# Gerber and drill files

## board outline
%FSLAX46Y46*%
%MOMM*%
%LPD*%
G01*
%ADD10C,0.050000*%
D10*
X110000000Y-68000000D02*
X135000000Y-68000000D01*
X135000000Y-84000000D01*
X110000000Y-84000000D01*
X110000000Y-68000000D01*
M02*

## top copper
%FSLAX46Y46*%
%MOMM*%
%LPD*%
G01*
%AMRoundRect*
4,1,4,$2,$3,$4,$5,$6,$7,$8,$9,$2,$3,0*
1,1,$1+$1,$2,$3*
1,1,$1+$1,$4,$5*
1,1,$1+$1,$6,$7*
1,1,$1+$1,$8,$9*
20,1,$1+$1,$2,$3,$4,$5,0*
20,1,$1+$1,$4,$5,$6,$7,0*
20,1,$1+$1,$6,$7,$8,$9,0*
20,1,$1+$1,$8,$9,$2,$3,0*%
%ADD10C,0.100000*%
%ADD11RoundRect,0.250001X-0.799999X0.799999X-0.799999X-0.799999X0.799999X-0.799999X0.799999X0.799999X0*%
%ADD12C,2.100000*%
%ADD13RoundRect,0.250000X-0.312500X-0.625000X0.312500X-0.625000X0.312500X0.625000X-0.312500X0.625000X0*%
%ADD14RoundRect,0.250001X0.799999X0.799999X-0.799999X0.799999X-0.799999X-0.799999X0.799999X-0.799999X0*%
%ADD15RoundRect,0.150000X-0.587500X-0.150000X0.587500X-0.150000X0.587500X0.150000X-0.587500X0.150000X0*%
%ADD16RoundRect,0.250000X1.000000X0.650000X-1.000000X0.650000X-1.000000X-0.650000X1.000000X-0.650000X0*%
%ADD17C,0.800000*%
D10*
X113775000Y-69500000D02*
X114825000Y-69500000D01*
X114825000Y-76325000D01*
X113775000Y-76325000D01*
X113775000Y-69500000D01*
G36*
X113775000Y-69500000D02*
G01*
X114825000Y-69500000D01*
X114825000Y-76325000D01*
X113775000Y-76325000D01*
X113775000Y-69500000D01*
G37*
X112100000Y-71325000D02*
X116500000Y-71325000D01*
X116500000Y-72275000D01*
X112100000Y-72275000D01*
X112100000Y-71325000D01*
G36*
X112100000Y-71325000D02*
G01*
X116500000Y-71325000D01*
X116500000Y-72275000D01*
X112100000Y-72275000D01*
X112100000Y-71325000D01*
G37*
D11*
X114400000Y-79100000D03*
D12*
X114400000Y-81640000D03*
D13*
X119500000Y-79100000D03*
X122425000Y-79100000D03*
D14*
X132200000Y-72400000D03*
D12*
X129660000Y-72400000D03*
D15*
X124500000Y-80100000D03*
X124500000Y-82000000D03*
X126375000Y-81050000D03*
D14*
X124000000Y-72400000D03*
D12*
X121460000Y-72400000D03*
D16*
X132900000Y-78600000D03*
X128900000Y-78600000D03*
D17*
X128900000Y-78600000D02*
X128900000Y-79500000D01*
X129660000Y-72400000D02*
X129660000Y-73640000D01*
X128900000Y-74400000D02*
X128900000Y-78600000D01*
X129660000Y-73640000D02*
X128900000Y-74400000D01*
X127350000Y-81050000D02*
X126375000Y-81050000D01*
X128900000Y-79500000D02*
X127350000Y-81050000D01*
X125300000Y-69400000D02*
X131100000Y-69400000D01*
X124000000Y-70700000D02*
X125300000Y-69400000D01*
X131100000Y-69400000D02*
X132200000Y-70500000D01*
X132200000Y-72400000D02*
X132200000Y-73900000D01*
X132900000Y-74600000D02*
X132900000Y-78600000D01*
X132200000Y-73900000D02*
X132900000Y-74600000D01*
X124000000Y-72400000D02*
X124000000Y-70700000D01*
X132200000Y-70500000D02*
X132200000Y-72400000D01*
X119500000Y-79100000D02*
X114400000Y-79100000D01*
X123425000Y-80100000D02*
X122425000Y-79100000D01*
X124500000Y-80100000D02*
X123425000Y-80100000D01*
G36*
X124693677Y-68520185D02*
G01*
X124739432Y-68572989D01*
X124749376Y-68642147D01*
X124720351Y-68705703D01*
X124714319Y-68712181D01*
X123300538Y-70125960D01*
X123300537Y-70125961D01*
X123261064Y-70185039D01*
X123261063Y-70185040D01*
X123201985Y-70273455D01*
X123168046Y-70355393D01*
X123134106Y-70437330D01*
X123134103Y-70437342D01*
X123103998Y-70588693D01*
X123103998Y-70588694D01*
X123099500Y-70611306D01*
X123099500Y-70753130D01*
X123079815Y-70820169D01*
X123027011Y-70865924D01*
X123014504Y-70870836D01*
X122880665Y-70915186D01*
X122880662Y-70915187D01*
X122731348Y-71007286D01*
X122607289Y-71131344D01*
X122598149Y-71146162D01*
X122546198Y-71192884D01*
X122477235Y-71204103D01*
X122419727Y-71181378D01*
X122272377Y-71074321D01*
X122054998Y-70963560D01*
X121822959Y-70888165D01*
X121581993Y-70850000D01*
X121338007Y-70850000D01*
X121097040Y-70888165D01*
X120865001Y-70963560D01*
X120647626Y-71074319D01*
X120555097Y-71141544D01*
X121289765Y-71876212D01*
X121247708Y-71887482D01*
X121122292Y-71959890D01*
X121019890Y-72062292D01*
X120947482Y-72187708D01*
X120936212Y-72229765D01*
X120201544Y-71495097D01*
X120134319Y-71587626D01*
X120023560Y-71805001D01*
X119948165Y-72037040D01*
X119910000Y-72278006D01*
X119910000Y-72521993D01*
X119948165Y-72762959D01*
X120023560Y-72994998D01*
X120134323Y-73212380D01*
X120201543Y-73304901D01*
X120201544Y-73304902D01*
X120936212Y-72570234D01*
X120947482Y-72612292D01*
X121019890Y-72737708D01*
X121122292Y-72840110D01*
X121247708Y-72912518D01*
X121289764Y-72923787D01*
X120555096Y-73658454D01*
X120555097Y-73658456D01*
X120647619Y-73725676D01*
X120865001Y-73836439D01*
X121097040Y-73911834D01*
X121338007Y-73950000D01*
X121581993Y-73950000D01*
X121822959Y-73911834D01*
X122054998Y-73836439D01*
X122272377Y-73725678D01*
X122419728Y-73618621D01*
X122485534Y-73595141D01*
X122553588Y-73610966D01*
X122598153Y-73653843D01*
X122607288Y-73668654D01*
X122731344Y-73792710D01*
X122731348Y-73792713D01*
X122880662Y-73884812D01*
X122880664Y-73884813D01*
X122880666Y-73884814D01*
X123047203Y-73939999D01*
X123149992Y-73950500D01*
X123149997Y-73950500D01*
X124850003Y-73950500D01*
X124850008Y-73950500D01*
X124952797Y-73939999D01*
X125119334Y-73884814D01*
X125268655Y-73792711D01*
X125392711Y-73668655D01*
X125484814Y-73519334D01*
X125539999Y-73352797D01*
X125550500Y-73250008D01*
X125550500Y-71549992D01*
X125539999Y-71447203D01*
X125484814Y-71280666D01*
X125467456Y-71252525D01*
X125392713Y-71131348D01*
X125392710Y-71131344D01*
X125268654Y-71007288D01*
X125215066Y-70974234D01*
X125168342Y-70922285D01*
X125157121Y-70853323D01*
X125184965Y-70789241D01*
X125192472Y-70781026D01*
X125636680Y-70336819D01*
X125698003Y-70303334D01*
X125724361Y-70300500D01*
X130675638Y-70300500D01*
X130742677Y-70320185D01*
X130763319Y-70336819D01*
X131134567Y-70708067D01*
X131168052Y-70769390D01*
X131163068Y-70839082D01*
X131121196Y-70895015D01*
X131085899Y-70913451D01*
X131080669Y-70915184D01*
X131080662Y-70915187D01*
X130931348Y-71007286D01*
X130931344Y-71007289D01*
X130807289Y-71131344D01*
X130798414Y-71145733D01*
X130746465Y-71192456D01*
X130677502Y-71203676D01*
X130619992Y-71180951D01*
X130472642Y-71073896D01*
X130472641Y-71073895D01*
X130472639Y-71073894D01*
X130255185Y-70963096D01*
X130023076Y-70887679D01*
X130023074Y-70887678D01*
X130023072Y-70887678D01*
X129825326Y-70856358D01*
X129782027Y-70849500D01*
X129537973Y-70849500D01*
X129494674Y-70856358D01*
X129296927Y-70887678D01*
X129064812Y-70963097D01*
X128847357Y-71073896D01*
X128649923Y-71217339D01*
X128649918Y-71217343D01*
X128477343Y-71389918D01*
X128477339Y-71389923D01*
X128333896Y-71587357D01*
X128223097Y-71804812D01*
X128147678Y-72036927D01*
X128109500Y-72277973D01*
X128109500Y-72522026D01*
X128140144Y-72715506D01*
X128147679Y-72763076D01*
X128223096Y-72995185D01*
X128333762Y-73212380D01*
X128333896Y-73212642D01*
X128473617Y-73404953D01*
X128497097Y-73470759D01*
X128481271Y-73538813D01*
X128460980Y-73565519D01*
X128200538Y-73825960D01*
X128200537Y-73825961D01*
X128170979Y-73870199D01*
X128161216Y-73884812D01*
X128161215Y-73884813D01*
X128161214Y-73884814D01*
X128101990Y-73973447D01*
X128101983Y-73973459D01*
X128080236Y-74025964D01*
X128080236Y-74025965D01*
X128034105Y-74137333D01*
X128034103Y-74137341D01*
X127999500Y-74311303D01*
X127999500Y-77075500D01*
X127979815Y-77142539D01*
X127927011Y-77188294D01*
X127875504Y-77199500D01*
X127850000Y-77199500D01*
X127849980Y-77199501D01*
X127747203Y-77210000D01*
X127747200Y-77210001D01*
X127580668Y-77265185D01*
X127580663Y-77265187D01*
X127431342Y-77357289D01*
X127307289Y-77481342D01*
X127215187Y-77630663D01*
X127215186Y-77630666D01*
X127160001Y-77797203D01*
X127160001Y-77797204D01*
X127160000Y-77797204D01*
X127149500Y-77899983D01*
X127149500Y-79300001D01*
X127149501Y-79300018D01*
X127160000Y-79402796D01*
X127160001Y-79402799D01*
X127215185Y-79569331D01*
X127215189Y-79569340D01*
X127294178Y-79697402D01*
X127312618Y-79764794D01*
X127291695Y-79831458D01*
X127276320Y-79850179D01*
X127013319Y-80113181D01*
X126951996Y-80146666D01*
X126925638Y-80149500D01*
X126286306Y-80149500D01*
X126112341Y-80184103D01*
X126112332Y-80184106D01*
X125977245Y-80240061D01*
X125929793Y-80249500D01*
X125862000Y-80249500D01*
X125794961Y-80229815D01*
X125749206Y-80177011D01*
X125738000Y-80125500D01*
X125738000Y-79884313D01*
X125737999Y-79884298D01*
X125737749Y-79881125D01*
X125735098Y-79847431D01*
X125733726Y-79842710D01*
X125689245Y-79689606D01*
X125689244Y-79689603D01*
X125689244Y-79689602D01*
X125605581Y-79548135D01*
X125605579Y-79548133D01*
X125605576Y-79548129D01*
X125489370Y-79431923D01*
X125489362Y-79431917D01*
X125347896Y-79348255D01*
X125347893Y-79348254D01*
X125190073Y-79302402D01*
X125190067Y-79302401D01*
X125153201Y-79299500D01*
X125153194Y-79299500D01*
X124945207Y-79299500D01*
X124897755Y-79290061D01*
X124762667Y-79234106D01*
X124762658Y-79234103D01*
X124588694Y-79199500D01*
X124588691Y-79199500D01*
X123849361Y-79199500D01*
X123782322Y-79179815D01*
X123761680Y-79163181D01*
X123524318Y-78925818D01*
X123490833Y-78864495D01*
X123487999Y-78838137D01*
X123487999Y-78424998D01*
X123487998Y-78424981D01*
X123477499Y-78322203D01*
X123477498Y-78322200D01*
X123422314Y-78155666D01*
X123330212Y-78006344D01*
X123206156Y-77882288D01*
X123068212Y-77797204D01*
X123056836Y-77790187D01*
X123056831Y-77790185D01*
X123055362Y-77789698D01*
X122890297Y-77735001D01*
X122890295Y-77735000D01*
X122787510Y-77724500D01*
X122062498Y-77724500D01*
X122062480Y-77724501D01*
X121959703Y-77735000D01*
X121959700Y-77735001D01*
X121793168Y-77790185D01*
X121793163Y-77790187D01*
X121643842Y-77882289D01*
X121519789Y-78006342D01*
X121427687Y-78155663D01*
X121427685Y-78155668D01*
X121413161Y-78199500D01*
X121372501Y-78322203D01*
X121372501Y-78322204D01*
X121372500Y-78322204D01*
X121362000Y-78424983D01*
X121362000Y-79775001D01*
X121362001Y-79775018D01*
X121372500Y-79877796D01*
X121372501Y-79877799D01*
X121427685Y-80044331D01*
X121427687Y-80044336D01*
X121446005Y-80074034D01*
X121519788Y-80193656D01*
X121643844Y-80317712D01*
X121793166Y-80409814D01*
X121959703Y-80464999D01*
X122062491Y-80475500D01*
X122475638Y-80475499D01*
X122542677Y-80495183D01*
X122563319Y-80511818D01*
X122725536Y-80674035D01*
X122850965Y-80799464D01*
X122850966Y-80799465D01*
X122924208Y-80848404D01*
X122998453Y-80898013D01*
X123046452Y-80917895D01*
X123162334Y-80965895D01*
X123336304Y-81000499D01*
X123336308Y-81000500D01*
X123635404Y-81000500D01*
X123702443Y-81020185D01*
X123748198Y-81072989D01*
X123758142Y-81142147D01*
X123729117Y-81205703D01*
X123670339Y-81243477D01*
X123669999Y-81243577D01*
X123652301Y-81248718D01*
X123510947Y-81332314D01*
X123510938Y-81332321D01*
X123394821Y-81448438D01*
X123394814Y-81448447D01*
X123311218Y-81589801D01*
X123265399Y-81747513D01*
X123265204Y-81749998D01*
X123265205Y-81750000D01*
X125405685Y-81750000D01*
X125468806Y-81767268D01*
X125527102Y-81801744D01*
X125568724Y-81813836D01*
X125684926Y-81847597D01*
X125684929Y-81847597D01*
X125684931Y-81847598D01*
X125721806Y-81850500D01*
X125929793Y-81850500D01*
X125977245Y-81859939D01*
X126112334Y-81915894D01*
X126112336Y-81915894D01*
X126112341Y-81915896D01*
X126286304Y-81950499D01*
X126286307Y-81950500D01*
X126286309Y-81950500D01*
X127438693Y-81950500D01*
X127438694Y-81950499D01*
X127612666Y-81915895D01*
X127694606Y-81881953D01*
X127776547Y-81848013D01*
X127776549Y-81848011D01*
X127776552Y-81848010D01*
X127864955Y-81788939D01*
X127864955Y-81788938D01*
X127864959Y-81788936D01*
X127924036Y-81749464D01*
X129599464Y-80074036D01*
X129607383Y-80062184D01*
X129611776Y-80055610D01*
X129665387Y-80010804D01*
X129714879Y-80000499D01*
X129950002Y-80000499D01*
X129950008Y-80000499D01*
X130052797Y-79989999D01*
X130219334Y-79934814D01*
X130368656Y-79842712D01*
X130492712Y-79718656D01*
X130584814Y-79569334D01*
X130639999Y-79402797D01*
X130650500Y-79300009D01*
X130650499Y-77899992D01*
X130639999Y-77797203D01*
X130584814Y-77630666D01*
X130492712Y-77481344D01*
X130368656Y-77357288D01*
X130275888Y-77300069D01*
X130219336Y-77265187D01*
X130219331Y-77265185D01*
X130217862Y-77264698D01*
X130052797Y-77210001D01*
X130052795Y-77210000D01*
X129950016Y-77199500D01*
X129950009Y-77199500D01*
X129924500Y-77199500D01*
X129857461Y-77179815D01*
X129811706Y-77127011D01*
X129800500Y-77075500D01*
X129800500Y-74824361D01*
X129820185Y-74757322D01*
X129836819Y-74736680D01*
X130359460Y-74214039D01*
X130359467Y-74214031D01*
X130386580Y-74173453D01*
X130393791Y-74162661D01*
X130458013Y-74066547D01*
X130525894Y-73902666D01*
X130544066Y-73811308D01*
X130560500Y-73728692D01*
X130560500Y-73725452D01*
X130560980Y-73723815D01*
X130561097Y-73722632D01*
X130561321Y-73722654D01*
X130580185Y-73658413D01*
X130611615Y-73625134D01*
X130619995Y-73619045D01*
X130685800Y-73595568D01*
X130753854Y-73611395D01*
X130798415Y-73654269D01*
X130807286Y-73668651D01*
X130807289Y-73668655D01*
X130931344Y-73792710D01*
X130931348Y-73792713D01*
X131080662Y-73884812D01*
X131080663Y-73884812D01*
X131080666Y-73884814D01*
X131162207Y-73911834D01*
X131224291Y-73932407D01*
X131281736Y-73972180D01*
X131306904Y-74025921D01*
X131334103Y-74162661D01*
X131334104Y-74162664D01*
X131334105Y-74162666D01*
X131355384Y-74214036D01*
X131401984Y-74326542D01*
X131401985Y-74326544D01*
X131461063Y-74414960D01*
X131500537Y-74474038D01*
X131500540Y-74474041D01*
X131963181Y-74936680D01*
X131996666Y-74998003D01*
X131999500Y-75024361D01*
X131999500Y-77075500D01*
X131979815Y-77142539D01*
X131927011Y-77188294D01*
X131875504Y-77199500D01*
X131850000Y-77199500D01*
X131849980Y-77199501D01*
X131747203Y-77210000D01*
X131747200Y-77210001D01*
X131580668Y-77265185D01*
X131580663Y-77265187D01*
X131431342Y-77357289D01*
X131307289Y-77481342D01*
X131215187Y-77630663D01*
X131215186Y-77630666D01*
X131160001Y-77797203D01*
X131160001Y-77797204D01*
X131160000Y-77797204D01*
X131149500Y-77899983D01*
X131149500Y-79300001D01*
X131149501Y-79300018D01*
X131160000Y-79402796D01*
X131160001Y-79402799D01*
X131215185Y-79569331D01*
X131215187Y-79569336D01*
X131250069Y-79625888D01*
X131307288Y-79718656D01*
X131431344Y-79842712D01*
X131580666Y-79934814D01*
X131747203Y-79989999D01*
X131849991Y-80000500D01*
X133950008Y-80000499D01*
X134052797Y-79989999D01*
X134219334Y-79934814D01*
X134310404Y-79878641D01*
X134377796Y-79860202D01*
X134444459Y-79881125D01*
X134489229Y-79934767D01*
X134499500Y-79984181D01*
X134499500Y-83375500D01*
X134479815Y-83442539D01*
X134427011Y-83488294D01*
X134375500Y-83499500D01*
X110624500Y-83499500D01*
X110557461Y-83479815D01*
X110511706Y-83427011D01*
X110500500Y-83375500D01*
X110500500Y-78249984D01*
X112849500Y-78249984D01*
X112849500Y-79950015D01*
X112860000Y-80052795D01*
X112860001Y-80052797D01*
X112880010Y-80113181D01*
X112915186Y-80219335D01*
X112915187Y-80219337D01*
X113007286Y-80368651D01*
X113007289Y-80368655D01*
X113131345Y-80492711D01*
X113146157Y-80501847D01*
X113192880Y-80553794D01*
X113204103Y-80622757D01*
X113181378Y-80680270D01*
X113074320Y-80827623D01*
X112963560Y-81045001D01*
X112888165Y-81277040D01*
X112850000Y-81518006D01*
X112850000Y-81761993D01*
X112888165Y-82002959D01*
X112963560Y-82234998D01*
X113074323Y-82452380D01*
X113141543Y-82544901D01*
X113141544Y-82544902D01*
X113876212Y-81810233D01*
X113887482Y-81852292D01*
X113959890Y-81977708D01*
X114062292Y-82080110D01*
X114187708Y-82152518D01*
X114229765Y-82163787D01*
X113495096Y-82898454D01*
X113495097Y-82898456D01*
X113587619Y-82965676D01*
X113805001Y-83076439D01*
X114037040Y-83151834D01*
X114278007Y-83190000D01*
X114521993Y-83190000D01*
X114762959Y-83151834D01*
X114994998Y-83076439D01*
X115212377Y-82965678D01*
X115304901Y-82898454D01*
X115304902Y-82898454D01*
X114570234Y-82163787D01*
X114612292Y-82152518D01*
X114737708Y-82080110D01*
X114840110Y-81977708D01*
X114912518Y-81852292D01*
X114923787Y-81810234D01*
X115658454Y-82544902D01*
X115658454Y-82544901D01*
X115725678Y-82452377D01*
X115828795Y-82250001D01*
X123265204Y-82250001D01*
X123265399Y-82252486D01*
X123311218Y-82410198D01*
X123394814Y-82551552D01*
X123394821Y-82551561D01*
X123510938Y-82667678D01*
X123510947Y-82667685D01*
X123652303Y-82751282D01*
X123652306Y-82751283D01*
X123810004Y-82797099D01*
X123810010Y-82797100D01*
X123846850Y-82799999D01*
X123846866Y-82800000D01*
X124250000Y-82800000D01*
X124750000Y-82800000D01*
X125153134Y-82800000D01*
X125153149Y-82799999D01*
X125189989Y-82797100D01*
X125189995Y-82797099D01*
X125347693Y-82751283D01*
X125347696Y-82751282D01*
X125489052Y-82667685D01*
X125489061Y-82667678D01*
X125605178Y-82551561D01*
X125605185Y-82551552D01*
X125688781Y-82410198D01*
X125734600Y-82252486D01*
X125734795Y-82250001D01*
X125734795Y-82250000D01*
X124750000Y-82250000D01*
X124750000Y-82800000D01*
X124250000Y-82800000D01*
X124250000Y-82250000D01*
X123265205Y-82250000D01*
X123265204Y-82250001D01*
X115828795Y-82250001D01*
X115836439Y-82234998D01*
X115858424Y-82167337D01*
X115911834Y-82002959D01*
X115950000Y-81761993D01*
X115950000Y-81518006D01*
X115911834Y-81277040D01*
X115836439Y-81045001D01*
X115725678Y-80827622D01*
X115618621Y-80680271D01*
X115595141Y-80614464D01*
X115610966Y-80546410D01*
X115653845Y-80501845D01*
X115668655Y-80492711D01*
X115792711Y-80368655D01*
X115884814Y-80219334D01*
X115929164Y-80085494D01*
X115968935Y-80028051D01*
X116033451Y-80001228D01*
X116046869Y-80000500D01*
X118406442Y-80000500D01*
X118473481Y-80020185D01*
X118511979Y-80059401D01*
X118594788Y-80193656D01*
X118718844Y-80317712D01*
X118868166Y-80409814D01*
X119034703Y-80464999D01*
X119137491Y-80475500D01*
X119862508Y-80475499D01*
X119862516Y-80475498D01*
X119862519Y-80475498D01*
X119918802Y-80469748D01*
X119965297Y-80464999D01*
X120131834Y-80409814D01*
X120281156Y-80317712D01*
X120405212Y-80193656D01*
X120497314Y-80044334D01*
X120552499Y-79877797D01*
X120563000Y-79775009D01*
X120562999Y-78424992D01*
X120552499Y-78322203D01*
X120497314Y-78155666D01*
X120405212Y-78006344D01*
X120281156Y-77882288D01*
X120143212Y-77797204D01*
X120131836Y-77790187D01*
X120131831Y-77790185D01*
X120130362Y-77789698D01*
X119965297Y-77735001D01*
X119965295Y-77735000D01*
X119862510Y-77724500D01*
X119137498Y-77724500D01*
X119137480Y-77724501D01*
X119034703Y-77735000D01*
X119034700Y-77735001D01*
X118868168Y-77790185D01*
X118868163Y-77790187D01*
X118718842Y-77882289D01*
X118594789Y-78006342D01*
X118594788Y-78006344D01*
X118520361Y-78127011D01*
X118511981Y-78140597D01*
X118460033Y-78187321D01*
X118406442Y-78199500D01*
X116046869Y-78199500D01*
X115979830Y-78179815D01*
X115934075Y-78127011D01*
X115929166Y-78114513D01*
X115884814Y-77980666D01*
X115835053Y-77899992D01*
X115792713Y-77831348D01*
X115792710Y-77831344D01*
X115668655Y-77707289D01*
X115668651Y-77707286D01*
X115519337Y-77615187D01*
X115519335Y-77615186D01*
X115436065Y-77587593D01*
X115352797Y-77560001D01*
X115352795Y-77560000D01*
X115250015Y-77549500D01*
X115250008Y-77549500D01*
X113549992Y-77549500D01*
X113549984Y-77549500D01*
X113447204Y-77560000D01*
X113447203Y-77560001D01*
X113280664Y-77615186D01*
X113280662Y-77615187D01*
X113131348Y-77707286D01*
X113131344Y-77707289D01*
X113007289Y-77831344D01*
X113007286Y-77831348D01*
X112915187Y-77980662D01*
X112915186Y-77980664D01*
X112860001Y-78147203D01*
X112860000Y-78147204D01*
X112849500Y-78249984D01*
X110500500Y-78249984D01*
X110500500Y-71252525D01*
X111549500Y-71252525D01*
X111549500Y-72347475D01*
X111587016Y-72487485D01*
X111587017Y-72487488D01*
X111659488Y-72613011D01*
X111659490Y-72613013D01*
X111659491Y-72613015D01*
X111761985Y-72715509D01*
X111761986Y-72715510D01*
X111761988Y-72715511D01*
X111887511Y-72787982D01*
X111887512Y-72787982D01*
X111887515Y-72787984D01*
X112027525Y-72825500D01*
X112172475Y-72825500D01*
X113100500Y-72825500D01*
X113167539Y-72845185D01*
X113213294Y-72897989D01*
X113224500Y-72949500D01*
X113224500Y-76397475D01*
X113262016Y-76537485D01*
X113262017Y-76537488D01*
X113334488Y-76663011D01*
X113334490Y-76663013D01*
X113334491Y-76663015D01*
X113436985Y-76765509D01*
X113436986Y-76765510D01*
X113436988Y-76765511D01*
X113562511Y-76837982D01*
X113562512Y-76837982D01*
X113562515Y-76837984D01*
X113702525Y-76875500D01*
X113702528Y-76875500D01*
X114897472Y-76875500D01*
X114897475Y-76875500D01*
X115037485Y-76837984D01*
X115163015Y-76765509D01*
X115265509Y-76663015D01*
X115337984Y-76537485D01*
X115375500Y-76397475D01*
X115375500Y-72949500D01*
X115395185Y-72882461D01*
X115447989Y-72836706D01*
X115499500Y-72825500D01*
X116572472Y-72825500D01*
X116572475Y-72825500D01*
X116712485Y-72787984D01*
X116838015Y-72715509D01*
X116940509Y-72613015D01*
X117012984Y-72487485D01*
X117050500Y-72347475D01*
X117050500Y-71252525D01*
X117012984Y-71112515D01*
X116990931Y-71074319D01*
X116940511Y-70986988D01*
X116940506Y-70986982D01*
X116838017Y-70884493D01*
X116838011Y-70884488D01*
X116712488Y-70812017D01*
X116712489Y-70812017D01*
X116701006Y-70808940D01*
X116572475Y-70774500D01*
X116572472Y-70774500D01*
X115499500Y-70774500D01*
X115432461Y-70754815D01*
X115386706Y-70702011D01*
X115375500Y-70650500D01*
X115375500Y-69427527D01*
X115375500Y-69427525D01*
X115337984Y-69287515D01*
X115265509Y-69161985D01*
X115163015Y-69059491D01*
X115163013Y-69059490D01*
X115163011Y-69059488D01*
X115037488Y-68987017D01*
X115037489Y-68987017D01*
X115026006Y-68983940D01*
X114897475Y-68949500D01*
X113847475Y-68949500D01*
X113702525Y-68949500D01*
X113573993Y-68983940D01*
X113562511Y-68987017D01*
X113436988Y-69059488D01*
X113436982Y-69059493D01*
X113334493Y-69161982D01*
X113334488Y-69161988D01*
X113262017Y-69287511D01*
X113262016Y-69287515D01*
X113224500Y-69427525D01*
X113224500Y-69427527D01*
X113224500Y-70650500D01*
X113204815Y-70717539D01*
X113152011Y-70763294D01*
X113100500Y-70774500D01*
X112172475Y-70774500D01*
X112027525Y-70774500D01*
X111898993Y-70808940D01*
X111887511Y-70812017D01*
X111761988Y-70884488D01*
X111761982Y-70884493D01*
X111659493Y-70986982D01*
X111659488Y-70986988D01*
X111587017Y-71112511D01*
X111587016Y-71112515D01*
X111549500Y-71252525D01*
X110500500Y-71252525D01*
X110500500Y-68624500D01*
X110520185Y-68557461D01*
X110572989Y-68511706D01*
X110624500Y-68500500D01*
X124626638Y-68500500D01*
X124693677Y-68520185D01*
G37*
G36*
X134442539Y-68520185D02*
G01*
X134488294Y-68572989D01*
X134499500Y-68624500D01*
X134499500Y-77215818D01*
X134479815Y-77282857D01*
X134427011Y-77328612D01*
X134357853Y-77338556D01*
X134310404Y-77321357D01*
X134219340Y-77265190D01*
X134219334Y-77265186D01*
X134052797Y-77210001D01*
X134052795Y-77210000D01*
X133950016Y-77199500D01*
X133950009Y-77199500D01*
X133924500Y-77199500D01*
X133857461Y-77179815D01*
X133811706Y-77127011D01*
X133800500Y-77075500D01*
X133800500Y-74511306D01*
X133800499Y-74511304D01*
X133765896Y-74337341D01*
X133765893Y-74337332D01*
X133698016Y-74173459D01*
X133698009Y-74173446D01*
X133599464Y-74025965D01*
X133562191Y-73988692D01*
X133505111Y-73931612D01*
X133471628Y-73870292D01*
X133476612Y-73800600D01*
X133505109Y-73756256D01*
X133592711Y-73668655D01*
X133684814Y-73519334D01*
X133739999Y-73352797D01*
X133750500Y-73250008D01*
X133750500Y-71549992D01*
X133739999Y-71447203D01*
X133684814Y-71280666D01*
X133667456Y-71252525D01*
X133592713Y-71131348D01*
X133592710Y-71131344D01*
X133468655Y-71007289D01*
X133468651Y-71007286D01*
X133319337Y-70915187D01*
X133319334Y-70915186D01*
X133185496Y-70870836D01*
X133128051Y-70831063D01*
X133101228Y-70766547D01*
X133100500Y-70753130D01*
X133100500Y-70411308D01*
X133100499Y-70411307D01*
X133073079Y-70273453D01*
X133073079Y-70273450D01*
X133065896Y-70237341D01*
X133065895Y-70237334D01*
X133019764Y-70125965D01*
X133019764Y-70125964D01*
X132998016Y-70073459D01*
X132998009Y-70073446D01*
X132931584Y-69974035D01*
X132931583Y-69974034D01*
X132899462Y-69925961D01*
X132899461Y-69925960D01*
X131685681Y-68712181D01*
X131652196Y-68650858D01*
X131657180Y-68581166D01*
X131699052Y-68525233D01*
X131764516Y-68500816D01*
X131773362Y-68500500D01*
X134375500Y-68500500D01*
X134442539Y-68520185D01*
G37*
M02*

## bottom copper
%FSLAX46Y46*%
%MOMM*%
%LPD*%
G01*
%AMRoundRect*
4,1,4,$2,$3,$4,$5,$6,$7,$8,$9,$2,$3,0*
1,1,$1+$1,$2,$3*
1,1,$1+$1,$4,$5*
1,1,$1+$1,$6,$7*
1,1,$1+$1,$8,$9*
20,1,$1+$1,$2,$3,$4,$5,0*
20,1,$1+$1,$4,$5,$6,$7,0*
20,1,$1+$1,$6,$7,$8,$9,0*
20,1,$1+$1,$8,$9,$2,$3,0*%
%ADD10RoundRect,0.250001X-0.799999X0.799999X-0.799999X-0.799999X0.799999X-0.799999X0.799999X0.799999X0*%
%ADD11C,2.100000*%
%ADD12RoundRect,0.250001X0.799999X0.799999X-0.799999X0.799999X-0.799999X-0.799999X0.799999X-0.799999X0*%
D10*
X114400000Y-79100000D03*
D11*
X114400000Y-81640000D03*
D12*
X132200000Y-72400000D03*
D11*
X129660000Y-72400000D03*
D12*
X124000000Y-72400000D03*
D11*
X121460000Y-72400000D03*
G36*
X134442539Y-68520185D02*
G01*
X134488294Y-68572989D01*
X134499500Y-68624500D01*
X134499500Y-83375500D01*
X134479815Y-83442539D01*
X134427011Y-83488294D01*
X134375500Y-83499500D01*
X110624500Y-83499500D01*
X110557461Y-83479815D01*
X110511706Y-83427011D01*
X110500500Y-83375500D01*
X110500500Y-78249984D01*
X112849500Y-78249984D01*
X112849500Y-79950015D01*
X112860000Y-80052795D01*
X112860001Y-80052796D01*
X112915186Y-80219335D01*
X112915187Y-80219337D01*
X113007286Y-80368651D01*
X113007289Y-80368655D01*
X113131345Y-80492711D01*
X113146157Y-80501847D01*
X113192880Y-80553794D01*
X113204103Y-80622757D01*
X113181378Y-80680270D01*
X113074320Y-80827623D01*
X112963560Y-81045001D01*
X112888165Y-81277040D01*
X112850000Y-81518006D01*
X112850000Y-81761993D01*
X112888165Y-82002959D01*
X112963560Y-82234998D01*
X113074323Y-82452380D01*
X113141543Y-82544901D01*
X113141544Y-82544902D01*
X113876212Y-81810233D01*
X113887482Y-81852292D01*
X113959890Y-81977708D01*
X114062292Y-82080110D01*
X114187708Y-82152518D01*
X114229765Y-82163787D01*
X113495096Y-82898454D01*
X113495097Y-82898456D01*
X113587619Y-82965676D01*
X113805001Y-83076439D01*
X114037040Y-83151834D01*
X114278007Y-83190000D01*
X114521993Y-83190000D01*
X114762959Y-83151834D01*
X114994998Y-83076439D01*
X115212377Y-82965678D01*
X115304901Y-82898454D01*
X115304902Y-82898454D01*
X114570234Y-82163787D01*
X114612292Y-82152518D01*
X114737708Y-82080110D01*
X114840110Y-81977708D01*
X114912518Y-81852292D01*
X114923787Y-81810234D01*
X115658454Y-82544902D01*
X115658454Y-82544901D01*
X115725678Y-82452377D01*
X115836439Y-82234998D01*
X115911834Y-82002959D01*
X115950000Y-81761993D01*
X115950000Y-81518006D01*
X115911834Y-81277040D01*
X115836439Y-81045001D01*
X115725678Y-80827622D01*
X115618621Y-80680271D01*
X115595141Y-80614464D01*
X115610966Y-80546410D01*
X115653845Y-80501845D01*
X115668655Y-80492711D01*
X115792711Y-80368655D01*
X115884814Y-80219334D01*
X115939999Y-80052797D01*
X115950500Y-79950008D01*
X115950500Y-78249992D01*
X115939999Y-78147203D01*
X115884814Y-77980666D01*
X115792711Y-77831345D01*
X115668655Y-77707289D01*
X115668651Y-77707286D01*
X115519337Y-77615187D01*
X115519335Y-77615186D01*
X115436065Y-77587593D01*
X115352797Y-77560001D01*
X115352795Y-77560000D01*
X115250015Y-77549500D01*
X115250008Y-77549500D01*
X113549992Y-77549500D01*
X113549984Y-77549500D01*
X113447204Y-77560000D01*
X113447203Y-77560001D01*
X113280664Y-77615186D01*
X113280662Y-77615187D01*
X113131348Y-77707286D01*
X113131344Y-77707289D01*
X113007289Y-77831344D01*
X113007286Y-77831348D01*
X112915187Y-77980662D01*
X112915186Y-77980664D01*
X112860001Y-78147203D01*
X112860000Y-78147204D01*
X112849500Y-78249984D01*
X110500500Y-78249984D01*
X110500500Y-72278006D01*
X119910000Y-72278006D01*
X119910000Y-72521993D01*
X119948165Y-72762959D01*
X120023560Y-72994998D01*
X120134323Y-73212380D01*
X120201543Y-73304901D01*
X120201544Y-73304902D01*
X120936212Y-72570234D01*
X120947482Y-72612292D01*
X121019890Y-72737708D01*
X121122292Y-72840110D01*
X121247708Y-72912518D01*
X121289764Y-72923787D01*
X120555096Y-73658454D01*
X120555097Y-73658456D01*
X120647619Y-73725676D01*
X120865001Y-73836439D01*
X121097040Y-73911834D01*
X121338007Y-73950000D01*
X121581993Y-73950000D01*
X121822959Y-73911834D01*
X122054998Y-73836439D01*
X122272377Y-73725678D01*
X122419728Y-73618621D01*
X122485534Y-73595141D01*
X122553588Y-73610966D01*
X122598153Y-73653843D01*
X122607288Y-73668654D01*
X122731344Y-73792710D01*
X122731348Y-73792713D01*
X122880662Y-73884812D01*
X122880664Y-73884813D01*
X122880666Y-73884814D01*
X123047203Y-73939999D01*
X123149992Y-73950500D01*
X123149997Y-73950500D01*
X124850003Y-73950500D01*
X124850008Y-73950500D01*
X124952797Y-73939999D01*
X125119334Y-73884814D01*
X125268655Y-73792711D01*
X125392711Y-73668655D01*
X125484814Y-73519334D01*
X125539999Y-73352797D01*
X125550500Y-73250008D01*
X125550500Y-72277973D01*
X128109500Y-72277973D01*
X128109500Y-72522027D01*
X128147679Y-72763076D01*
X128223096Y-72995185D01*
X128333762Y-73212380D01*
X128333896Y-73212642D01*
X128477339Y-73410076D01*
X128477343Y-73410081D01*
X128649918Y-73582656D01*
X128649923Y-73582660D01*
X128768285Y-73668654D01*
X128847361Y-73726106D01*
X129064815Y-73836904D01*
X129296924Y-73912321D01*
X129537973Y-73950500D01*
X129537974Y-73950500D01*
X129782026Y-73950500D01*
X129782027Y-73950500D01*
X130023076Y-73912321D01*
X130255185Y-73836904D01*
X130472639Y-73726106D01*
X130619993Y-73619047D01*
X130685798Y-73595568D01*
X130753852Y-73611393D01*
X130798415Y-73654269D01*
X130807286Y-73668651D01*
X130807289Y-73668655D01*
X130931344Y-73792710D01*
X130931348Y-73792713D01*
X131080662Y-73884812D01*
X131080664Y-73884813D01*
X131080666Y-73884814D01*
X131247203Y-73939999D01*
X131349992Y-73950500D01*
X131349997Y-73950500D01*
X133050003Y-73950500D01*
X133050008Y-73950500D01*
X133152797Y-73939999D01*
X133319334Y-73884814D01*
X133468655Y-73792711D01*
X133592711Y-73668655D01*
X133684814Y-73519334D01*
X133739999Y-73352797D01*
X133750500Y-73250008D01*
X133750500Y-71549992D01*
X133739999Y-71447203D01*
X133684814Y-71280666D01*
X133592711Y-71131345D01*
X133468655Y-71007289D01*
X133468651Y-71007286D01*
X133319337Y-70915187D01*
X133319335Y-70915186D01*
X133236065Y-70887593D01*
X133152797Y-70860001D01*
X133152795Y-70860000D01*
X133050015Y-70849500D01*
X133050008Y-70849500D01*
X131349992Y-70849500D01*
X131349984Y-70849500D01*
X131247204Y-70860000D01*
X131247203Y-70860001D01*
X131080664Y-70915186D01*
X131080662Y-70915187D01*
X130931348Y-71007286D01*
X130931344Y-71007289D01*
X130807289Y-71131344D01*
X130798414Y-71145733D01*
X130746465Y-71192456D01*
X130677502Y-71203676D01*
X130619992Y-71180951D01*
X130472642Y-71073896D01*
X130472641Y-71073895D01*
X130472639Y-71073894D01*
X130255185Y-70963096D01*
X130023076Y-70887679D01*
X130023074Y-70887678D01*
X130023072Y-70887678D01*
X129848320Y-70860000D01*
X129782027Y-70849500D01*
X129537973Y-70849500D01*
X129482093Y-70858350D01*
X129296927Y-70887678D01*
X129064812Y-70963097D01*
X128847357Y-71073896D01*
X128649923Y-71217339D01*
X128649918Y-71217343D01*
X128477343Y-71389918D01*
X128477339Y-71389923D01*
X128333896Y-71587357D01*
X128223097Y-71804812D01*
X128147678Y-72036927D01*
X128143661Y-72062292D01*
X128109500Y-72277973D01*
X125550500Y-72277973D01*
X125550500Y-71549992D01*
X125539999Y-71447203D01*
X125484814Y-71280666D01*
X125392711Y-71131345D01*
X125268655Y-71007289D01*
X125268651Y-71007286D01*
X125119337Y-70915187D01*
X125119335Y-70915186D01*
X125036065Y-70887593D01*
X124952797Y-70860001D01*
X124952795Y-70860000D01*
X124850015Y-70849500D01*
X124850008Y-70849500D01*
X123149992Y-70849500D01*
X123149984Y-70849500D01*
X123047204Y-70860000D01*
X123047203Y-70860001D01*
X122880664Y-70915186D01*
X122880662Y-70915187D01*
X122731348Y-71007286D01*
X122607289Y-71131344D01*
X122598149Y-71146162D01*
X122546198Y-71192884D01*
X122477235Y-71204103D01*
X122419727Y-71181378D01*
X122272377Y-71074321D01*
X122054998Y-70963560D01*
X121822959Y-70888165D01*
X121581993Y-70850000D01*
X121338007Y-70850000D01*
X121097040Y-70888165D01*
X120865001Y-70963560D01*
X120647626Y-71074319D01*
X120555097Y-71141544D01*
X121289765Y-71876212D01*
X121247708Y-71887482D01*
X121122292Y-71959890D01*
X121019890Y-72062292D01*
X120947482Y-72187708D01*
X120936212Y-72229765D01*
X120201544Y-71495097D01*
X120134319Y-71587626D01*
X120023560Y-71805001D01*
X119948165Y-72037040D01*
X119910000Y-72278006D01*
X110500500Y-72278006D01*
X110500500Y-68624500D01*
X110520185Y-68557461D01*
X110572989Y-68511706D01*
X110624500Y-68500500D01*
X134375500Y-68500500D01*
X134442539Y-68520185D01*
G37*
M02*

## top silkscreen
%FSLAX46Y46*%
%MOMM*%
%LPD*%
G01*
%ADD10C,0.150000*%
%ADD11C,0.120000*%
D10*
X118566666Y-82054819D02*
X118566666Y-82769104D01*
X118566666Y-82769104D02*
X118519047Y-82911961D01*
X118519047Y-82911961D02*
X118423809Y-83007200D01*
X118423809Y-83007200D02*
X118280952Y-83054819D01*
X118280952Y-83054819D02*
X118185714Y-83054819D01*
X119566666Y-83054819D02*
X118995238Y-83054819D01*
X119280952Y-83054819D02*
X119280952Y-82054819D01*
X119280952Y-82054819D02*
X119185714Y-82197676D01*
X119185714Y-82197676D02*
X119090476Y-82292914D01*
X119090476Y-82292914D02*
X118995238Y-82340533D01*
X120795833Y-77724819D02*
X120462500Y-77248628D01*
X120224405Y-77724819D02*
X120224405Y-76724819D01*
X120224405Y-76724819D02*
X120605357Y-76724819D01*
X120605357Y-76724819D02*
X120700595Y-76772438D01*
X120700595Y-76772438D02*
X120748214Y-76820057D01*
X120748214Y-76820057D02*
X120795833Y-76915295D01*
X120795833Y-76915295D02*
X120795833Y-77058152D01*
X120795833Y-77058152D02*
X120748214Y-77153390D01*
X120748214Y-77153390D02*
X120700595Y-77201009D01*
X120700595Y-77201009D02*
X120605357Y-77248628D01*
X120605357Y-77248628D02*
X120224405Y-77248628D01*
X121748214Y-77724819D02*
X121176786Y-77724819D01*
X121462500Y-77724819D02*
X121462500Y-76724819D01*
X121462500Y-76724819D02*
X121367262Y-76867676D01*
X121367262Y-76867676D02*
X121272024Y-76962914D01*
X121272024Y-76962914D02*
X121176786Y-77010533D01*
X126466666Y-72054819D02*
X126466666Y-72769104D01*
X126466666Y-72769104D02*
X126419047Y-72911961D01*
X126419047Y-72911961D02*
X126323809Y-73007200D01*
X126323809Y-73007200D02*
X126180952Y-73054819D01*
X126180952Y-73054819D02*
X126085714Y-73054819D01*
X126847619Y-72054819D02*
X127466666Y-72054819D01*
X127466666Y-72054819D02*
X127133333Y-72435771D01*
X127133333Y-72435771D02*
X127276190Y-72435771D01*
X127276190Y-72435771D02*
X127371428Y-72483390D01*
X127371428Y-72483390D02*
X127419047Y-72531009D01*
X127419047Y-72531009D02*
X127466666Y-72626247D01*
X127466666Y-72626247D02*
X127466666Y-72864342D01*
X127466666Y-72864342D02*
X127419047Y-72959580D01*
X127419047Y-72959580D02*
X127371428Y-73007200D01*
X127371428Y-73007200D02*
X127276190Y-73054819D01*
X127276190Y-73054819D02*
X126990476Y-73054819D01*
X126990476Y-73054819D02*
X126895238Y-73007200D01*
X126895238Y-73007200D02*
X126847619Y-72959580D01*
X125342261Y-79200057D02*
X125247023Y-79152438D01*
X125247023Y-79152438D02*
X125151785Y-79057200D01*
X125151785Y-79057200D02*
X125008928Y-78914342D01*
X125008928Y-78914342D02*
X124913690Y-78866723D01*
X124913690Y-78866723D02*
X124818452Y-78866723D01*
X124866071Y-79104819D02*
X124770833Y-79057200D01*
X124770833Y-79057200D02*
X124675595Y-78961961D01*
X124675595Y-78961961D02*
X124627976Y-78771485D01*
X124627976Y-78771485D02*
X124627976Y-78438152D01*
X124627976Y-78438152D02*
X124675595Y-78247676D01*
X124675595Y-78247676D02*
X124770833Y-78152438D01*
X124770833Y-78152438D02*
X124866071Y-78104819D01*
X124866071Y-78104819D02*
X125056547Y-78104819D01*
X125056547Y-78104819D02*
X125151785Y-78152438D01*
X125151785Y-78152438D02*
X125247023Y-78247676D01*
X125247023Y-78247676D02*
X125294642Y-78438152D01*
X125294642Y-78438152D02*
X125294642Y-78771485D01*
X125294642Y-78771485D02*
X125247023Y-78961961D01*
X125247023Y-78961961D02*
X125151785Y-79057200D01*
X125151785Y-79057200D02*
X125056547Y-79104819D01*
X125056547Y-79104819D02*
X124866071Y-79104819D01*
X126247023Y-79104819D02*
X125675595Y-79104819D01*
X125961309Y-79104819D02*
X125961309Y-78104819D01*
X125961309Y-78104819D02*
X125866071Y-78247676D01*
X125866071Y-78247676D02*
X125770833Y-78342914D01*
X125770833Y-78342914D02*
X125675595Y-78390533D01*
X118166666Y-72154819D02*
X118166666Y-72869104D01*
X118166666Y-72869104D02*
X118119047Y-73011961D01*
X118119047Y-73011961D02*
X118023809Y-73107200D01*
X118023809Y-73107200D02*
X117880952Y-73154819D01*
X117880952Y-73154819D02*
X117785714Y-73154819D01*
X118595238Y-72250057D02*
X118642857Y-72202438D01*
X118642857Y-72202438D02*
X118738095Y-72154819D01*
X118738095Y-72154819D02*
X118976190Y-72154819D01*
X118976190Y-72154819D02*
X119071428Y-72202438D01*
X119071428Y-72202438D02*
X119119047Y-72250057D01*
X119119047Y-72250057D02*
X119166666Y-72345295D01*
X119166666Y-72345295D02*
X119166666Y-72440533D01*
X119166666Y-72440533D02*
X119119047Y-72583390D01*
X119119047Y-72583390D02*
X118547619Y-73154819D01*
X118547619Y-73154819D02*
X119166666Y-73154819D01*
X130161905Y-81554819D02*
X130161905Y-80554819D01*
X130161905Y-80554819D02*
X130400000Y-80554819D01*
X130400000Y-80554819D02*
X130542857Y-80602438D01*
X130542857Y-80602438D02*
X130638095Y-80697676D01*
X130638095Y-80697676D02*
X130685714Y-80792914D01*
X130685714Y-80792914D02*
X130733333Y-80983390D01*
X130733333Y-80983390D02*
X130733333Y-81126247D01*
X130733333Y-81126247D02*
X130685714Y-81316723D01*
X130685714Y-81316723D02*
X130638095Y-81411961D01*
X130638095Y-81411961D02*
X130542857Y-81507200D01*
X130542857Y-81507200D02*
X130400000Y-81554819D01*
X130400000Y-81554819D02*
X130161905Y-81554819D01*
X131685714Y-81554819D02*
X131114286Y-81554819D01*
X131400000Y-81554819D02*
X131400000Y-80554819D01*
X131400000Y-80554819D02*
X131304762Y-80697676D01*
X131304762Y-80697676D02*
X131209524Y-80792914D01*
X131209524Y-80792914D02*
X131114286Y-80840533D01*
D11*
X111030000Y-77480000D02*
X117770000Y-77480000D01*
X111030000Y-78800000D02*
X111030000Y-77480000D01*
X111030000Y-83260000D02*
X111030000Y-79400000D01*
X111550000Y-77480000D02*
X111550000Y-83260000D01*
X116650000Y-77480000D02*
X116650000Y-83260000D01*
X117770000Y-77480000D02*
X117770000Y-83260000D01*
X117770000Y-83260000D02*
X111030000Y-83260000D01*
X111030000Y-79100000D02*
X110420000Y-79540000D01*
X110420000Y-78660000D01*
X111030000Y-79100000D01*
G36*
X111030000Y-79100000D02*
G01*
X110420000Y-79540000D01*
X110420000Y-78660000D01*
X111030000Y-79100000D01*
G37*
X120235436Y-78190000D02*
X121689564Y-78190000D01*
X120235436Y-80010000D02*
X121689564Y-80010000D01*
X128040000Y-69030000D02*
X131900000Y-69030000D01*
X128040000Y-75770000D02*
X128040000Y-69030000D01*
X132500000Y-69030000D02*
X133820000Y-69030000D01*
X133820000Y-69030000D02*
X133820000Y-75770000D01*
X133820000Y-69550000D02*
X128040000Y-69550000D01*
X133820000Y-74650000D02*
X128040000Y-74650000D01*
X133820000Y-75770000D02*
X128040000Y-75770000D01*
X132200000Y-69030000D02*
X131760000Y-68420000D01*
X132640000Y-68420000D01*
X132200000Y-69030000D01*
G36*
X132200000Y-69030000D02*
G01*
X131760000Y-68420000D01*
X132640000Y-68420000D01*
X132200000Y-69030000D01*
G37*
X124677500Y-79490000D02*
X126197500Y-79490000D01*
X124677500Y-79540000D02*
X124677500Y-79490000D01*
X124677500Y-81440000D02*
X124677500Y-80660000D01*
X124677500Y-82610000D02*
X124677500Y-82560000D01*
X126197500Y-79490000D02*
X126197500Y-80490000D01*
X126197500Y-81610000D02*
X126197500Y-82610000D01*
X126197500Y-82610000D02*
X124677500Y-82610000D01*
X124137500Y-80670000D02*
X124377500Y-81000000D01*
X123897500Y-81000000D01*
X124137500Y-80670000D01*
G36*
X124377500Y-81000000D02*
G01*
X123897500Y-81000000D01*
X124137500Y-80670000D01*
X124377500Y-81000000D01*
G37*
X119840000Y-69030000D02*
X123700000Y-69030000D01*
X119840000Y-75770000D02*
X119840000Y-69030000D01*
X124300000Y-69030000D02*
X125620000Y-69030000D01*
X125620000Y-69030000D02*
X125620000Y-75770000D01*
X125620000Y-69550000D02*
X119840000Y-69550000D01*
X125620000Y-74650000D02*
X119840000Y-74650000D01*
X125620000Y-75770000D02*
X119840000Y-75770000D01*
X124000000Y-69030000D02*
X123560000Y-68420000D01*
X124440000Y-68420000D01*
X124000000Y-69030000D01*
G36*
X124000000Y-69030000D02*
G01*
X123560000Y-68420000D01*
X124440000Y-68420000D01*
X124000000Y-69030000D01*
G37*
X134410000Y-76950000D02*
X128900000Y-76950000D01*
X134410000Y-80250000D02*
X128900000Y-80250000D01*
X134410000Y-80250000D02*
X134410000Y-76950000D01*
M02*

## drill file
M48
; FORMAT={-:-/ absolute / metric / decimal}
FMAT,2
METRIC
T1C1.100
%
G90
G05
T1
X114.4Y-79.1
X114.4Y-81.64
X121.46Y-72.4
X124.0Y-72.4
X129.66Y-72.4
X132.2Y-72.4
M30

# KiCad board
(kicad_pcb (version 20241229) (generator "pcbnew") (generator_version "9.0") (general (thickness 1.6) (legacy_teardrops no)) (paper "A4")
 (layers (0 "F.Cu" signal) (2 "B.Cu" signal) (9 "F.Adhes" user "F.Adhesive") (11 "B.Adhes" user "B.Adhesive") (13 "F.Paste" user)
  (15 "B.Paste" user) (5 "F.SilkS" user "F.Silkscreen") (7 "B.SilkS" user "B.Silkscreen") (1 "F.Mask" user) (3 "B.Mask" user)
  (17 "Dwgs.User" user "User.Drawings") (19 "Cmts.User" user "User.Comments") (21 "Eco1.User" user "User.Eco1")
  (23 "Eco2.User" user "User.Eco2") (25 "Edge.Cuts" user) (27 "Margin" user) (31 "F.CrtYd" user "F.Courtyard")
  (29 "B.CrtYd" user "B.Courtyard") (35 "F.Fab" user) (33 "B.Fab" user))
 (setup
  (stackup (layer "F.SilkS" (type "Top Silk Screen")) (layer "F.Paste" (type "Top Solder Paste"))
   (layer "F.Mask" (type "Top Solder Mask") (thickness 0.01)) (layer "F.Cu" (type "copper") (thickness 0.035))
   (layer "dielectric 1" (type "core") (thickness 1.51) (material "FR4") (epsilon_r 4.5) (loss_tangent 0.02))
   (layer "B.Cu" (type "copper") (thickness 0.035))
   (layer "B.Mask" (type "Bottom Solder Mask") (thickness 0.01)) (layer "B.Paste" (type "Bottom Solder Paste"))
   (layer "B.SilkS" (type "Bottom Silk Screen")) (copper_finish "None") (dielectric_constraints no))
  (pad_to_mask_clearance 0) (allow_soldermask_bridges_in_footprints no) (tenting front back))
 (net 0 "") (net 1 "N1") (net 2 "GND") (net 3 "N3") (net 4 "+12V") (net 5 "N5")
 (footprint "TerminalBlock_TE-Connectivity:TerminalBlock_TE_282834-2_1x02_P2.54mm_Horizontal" (layer "F.Cu") (at 114.4 79.1 -90)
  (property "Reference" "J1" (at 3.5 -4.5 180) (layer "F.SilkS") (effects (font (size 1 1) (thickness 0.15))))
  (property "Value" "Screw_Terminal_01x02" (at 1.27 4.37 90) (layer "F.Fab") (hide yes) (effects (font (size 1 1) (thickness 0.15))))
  (fp_line (start -1.62 3.37) (end -1.62 -3.37) (stroke (width 0.12) (type solid)) (layer "F.SilkS"))
  (fp_line (start -0.3 3.37) (end -1.62 3.37) (stroke (width 0.12) (type solid)) (layer "F.SilkS"))
  (fp_line (start 4.16 3.37) (end 0.3 3.37) (stroke (width 0.12) (type solid)) (layer "F.SilkS"))
  (fp_line (start -1.62 2.85) (end 4.16 2.85) (stroke (width 0.12) (type solid)) (layer "F.SilkS"))
  (fp_line (start -1.62 -2.25) (end 4.16 -2.25) (stroke (width 0.12) (type solid)) (layer "F.SilkS"))
  (fp_line (start -1.62 -3.37) (end 4.16 -3.37) (stroke (width 0.12) (type solid)) (layer "F.SilkS"))
  (fp_line (start 4.16 -3.37) (end 4.16 3.37) (stroke (width 0.12) (type solid)) (layer "F.SilkS"))
  (fp_poly (pts (xy 0 3.37) (xy 0.44 3.98) (xy -0.44 3.98)) (stroke (width 0.12) (type solid)) (fill yes) (layer "F.SilkS"))
  (pad "1" thru_hole roundrect (at 0 0 270) (size 2.1 2.1) (drill 1.1) (layers "*.Cu" "*.Mask") (remove_unused_layers no)
   (roundrect_rratio 0.119048) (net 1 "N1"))
  (pad "2" thru_hole circle (at 2.54 0 270) (size 2.1 2.1) (drill 1.1) (layers "*.Cu" "*.Mask") (remove_unused_layers no) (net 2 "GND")))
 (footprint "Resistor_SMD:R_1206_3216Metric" (layer "F.Cu") (at 120.9625 79.1)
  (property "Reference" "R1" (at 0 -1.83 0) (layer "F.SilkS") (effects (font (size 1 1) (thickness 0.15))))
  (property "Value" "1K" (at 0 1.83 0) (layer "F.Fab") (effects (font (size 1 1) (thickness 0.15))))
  (fp_line (start -0.727064 -0.91) (end 0.727064 -0.91) (stroke (width 0.12) (type solid)) (layer "F.SilkS"))
  (fp_line (start -0.727064 0.91) (end 0.727064 0.91) (stroke (width 0.12) (type solid)) (layer "F.SilkS"))
  (pad "1" smd roundrect (at -1.4625 0) (size 1.125 1.75) (layers "F.Cu" "F.Mask" "F.Paste") (roundrect_rratio 0.222222) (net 1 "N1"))
  (pad "2" smd roundrect (at 1.4625 0) (size 1.125 1.75) (layers "F.Cu" "F.Mask" "F.Paste") (roundrect_rratio 0.222222) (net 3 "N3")))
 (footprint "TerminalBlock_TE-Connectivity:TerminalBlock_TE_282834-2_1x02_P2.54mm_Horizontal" (layer "F.Cu") (at 132.2 72.4 180)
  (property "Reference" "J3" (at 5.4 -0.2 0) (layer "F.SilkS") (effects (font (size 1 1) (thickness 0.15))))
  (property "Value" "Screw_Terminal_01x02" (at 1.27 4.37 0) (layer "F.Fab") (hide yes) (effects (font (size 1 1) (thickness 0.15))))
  (fp_line (start 4.16 3.37) (end 0.3 3.37) (stroke (width 0.12) (type solid)) (layer "F.SilkS"))
  (fp_line (start 4.16 -3.37) (end 4.16 3.37) (stroke (width 0.12) (type solid)) (layer "F.SilkS"))
  (fp_line (start -0.3 3.37) (end -1.62 3.37) (stroke (width 0.12) (type solid)) (layer "F.SilkS"))
  (fp_line (start -1.62 3.37) (end -1.62 -3.37) (stroke (width 0.12) (type solid)) (layer "F.SilkS"))
  (fp_line (start -1.62 2.85) (end 4.16 2.85) (stroke (width 0.12) (type solid)) (layer "F.SilkS"))
  (fp_line (start -1.62 -2.25) (end 4.16 -2.25) (stroke (width 0.12) (type solid)) (layer "F.SilkS"))
  (fp_line (start -1.62 -3.37) (end 4.16 -3.37) (stroke (width 0.12) (type solid)) (layer "F.SilkS"))
  (fp_poly (pts (xy 0 3.37) (xy 0.44 3.98) (xy -0.44 3.98)) (stroke (width 0.12) (type solid)) (fill yes) (layer "F.SilkS"))
  (pad "1" thru_hole roundrect (at 0 0 180) (size 2.1 2.1) (drill 1.1) (layers "*.Cu" "*.Mask") (remove_unused_layers no)
   (roundrect_rratio 0.119048) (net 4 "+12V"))
  (pad "2" thru_hole circle (at 2.54 0 180) (size 2.1 2.1) (drill 1.1) (layers "*.Cu" "*.Mask") (remove_unused_layers no) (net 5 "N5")))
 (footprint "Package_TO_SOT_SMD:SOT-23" (layer "F.Cu") (at 125.4375 81.05)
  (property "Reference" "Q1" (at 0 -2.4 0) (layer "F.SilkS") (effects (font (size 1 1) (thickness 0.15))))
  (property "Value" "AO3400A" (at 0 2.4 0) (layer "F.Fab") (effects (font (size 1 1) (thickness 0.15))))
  (fp_line (start -0.76 -1.56) (end 0.76 -1.56) (stroke (width 0.12) (type solid)) (layer "F.SilkS"))
  (fp_line (start -0.76 -1.51) (end -0.76 -1.56) (stroke (width 0.12) (type solid)) (layer "F.SilkS"))
  (fp_line (start -0.76 0.39) (end -0.76 -0.39) (stroke (width 0.12) (type solid)) (layer "F.SilkS"))
  (fp_line (start -0.76 1.56) (end -0.76 1.51) (stroke (width 0.12) (type solid)) (layer "F.SilkS"))
  (fp_line (start 0.76 -1.56) (end 0.76 -0.56) (stroke (width 0.12) (type solid)) (layer "F.SilkS"))
  (fp_line (start 0.76 0.56) (end 0.76 1.56) (stroke (width 0.12) (type solid)) (layer "F.SilkS"))
  (fp_line (start 0.76 1.56) (end -0.76 1.56) (stroke (width 0.12) (type solid)) (layer "F.SilkS"))
  (fp_poly (pts (xy -1.3 -0.38) (xy -1.06 -0.05) (xy -1.54 -0.05)) (stroke (width 0.12) (type solid)) (fill yes) (layer "F.SilkS"))
  (pad "1" smd roundrect (at -0.9375 -0.95) (size 1.475 0.6) (layers "F.Cu" "F.Mask" "F.Paste") (roundrect_rratio 0.25) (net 3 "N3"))
  (pad "2" smd roundrect (at -0.9375 0.95) (size 1.475 0.6) (layers "F.Cu" "F.Mask" "F.Paste") (roundrect_rratio 0.25) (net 2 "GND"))
  (pad "3" smd roundrect (at 0.9375 0) (size 1.475 0.6) (layers "F.Cu" "F.Mask" "F.Paste") (roundrect_rratio 0.25) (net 5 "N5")))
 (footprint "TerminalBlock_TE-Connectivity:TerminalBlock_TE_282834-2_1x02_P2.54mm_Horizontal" (layer "F.Cu") (at 124 72.4 180)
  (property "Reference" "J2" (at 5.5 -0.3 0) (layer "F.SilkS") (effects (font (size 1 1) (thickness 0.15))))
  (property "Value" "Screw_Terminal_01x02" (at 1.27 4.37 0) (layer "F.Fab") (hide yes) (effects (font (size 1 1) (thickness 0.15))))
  (fp_line (start 4.16 3.37) (end 0.3 3.37) (stroke (width 0.12) (type solid)) (layer "F.SilkS"))
  (fp_line (start 4.16 -3.37) (end 4.16 3.37) (stroke (width 0.12) (type solid)) (layer "F.SilkS"))
  (fp_line (start -0.3 3.37) (end -1.62 3.37) (stroke (width 0.12) (type solid)) (layer "F.SilkS"))
  (fp_line (start -1.62 3.37) (end -1.62 -3.37) (stroke (width 0.12) (type solid)) (layer "F.SilkS"))
  (fp_line (start -1.62 2.85) (end 4.16 2.85) (stroke (width 0.12) (type solid)) (layer "F.SilkS"))
  (fp_line (start -1.62 -2.25) (end 4.16 -2.25) (stroke (width 0.12) (type solid)) (layer "F.SilkS"))
  (fp_line (start -1.62 -3.37) (end 4.16 -3.37) (stroke (width 0.12) (type solid)) (layer "F.SilkS"))
  (fp_poly (pts (xy 0 3.37) (xy 0.44 3.98) (xy -0.44 3.98)) (stroke (width 0.12) (type solid)) (fill yes) (layer "F.SilkS"))
  (pad "1" thru_hole roundrect (at 0 0 180) (size 2.1 2.1) (drill 1.1) (layers "*.Cu" "*.Mask") (remove_unused_layers no)
   (roundrect_rratio 0.119048) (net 4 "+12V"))
  (pad "2" thru_hole circle (at 2.54 0 180) (size 2.1 2.1) (drill 1.1) (layers "*.Cu" "*.Mask") (remove_unused_layers no) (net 2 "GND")))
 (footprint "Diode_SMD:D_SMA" (layer "F.Cu") (at 130.9 78.6 180)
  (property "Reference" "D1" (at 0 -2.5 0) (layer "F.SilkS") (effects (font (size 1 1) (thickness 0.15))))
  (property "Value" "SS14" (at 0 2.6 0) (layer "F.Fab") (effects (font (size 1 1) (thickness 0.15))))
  (fp_line (start -3.51 1.65) (end 2 1.65) (stroke (width 0.12) (type solid)) (layer "F.SilkS"))
  (fp_line (start -3.51 -1.65) (end 2 -1.65) (stroke (width 0.12) (type solid)) (layer "F.SilkS"))
  (fp_line (start -3.51 -1.65) (end -3.51 1.65) (stroke (width 0.12) (type solid)) (layer "F.SilkS"))
  (pad "1" smd roundrect (at -2 0 180) (size 2.5 1.8) (layers "F.Cu" "F.Mask" "F.Paste") (roundrect_rratio 0.1388888889) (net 4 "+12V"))
  (pad "2" smd roundrect (at 2 0 180) (size 2.5 1.8) (layers "F.Cu" "F.Mask" "F.Paste") (roundrect_rratio 0.1388888889) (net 5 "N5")))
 (gr_rect (start 113.775 69.5) (end 114.825 76.325) (stroke (width 0.1) (type solid)) (fill yes) (layer "F.Cu"))
 (gr_rect (start 112.1 71.325) (end 116.5 72.275) (stroke (width 0.1) (type solid)) (fill yes) (layer "F.Cu"))
 (gr_rect (start 110 68) (end 135 84) (stroke (width 0.05) (type default)) (fill no) (layer "Edge.Cuts"))
 (segment (start 128.9 78.6) (end 128.9 79.5) (width 0.8) (layer "F.Cu") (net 5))
 (segment (start 129.66 72.4) (end 129.66 73.64) (width 0.8) (layer "F.Cu") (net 5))
 (segment (start 128.9 74.4) (end 128.9 78.6) (width 0.8) (layer "F.Cu") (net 5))
 (segment (start 129.66 73.64) (end 128.9 74.4) (width 0.8) (layer "F.Cu") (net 5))
 (segment (start 127.35 81.05) (end 126.375 81.05) (width 0.8) (layer "F.Cu") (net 5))
 (segment (start 128.9 79.5) (end 127.35 81.05) (width 0.8) (layer "F.Cu") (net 5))
 (segment (start 125.3 69.4) (end 131.1 69.4) (width 0.8) (layer "F.Cu") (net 4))
 (segment (start 124 70.7) (end 125.3 69.4) (width 0.8) (layer "F.Cu") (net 4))
 (segment (start 131.1 69.4) (end 132.2 70.5) (width 0.8) (layer "F.Cu") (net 4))
 (segment (start 132.2 72.4) (end 132.2 73.9) (width 0.8) (layer "F.Cu") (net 4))
 (segment (start 132.9 74.6) (end 132.9 78.6) (width 0.8) (layer "F.Cu") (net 4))
 (segment (start 132.2 73.9) (end 132.9 74.6) (width 0.8) (layer "F.Cu") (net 4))
 (segment (start 124 72.4) (end 124 70.7) (width 0.8) (layer "F.Cu") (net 4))
 (segment (start 132.2 70.5) (end 132.2 72.4) (width 0.8) (layer "F.Cu") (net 4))
 (segment (start 119.5 79.1) (end 114.4 79.1) (width 0.8) (layer "F.Cu") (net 1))
 (segment (start 123.425 80.1) (end 122.425 79.1) (width 0.8) (layer "F.Cu") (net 3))
 (segment (start 124.5 80.1) (end 123.425 80.1) (width 0.8) (layer "F.Cu") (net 3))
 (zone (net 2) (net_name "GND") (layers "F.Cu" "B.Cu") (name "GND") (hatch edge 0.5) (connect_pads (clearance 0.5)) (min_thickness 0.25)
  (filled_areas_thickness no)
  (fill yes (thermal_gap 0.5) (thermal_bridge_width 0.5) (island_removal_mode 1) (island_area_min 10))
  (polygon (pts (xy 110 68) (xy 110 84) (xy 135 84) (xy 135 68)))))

